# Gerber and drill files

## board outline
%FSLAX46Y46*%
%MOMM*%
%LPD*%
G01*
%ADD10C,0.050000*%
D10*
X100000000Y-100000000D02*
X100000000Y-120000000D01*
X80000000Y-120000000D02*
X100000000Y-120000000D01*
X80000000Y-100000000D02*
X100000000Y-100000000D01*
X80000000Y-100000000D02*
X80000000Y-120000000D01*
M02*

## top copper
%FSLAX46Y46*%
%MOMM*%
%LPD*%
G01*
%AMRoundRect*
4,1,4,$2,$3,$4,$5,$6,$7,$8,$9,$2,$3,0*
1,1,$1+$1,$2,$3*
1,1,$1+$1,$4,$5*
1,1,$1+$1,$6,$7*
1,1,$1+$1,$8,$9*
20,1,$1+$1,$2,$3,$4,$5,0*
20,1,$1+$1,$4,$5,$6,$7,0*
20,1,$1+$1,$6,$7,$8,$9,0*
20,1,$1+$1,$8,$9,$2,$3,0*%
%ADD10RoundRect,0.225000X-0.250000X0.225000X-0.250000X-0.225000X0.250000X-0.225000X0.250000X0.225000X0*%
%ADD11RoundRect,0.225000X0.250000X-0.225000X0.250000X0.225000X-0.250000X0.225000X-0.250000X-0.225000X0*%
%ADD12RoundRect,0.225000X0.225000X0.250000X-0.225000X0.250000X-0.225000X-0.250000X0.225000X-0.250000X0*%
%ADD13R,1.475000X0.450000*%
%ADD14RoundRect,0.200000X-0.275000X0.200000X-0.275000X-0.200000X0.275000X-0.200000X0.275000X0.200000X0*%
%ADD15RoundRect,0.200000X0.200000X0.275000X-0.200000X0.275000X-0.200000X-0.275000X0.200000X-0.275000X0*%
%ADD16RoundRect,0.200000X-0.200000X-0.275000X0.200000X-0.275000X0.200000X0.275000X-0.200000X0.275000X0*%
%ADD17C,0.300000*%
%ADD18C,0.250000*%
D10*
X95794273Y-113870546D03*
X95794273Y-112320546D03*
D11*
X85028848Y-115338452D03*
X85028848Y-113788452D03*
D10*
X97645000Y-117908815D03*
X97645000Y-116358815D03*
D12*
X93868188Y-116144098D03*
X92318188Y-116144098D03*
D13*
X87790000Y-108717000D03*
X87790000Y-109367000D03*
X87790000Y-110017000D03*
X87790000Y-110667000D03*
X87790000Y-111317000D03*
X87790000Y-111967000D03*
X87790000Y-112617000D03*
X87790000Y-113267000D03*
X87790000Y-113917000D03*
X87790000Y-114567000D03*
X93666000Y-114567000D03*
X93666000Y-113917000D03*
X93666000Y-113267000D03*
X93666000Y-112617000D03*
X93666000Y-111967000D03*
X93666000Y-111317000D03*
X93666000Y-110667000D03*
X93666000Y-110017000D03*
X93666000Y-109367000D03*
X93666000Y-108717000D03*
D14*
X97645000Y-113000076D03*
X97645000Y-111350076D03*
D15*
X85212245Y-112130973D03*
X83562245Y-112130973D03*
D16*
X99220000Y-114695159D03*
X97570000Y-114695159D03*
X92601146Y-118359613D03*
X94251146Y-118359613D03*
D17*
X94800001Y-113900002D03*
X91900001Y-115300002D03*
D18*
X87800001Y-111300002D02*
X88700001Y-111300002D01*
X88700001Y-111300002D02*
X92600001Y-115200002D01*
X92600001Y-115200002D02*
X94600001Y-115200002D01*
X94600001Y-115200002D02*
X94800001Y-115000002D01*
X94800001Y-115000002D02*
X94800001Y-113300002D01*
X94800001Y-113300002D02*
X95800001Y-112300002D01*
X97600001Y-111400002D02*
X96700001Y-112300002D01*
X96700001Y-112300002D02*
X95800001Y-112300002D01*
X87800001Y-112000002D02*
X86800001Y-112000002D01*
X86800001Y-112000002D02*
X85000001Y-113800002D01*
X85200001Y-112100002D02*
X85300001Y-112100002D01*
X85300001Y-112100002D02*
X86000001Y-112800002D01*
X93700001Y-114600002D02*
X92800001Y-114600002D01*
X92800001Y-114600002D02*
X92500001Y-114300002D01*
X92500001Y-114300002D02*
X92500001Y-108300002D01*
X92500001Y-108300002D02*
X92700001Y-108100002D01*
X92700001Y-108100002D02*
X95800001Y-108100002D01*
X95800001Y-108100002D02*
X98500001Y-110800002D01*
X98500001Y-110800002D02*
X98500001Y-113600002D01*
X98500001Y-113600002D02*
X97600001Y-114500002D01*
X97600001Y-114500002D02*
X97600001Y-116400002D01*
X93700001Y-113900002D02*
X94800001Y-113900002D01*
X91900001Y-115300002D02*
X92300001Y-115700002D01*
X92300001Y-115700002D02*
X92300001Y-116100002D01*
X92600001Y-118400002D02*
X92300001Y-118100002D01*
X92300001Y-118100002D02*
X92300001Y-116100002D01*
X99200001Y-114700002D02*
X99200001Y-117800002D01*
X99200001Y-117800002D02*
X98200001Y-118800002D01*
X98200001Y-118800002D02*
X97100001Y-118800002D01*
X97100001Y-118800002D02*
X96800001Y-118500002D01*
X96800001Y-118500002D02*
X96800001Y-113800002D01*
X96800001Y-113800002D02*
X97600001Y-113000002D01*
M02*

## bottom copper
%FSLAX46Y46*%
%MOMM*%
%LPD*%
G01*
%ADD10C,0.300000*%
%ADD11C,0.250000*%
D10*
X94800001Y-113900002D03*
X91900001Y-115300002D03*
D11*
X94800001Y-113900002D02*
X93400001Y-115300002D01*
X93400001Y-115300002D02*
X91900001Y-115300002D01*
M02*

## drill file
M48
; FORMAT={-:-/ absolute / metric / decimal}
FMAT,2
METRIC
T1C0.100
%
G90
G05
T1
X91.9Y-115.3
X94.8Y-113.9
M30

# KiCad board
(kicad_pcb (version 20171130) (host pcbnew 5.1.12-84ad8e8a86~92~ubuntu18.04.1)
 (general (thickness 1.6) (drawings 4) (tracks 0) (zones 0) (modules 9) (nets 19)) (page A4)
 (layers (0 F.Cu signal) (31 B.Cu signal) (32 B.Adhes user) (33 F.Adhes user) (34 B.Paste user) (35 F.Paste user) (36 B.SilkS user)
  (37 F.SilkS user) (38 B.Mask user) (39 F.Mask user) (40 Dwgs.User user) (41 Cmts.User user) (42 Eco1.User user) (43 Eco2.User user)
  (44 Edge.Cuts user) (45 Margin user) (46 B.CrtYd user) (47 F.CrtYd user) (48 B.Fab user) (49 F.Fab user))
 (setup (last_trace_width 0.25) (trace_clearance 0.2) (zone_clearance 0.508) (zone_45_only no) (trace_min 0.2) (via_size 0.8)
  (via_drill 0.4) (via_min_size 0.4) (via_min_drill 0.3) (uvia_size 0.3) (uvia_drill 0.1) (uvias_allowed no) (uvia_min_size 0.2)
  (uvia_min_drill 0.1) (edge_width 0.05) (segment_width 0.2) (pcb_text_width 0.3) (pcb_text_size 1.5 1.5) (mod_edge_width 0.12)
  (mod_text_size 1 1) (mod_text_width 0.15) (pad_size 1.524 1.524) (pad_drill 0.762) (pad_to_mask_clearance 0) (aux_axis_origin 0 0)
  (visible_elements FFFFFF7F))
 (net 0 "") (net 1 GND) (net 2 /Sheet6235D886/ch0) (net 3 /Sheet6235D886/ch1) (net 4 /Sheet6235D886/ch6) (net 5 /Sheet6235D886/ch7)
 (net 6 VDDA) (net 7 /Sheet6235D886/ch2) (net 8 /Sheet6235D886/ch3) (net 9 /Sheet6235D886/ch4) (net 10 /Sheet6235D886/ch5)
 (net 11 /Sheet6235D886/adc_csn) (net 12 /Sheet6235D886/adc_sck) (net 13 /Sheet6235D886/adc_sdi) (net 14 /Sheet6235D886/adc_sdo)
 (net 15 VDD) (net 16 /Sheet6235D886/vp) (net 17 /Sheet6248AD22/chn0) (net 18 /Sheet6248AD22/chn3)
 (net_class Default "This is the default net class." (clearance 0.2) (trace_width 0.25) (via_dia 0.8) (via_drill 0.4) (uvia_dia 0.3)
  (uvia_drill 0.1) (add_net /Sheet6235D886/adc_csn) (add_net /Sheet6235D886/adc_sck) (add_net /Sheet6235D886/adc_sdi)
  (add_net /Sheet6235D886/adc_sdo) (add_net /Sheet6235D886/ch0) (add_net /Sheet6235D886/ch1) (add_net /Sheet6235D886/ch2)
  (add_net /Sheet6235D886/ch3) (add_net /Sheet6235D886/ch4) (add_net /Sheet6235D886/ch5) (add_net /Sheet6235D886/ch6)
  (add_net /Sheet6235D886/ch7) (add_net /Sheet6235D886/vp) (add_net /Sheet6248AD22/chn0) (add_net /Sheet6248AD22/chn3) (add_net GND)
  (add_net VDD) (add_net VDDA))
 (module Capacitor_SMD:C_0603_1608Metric (layer F.Cu) (at 95.794273 113.095546 270.000000)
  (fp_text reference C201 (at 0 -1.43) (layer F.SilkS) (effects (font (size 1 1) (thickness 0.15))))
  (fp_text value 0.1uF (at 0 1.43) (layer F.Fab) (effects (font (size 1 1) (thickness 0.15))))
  (pad 2 smd roundrect (at 0.775 0 270.000000) (size 0.9 0.95) (layers F.Cu F.Mask F.Paste) (roundrect_rratio 0.25) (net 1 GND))
  (pad 1 smd roundrect (at -0.775 0 270.000000) (size 0.9 0.95) (layers F.Cu F.Mask F.Paste) (roundrect_rratio 0.25)
   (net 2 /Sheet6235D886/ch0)))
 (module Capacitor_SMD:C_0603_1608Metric (layer F.Cu) (at 85.028848 114.563452 90.000000)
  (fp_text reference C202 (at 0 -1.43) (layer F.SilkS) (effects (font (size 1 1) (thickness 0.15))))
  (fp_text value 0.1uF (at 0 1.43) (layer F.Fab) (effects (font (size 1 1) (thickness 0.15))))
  (pad 1 smd roundrect (at -0.775 0 90.000000) (size 0.9 0.95) (layers F.Cu F.Mask F.Paste) (roundrect_rratio 0.25) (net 1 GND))
  (pad 2 smd roundrect (at 0.775 0 90.000000) (size 0.9 0.95) (layers F.Cu F.Mask F.Paste) (roundrect_rratio 0.25)
   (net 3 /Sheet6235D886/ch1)))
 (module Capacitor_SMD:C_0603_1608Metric (layer F.Cu) (at 97.645000 117.133815 270.000000)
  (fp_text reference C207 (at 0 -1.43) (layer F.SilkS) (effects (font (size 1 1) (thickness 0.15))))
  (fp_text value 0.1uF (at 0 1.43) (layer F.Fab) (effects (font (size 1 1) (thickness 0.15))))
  (pad 2 smd roundrect (at 0.775 0 270.000000) (size 0.9 0.95) (layers F.Cu F.Mask F.Paste) (roundrect_rratio 0.25) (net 1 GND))
  (pad 1 smd roundrect (at -0.775 0 270.000000) (size 0.9 0.95) (layers F.Cu F.Mask F.Paste) (roundrect_rratio 0.25)
   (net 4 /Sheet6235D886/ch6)))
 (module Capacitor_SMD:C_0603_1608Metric (layer F.Cu) (at 93.093188 116.144098 180.000000)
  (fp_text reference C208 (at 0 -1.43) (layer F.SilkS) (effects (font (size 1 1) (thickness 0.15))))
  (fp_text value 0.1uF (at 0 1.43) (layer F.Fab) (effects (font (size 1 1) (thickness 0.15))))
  (pad 1 smd roundrect (at -0.775 0 180.000000) (size 0.9 0.95) (layers F.Cu F.Mask F.Paste) (roundrect_rratio 0.25) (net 1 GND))
  (pad 2 smd roundrect (at 0.775 0 180.000000) (size 0.9 0.95) (layers F.Cu F.Mask F.Paste) (roundrect_rratio 0.25)
   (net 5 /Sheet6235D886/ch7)))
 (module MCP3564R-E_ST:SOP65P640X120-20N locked (layer F.Cu) (at 90.728000 111.642000)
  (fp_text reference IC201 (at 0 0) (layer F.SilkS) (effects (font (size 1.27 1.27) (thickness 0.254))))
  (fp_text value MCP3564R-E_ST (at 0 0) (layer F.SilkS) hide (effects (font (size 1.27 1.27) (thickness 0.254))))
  (pad 1 smd rect (at -2.938 -2.925 90.000000) (size 0.45 1.475) (layers F.Cu F.Mask F.Paste) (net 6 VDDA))
  (pad 2 smd rect (at -2.938 -2.275 90.000000) (size 0.45 1.475) (layers F.Cu F.Mask F.Paste) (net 1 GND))
  (pad 3 smd rect (at -2.938 -1.625 90.000000) (size 0.45 1.475) (layers F.Cu F.Mask F.Paste) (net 1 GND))
  (pad 4 smd rect (at -2.938 -0.975 90.000000) (size 0.45 1.475) (layers F.Cu F.Mask F.Paste))
  (pad 5 smd rect (at -2.938 -0.325 90.000000) (size 0.45 1.475) (layers F.Cu F.Mask F.Paste) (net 2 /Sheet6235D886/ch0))
  (pad 6 smd rect (at -2.938 0.325 90.000000) (size 0.45 1.475) (layers F.Cu F.Mask F.Paste) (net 3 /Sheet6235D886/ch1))
  (pad 7 smd rect (at -2.938 0.975 90.000000) (size 0.45 1.475) (layers F.Cu F.Mask F.Paste) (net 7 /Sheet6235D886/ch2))
  (pad 8 smd rect (at -2.938 1.625 90.000000) (size 0.45 1.475) (layers F.Cu F.Mask F.Paste) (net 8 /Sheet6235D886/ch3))
  (pad 9 smd rect (at -2.938 2.275 90.000000) (size 0.45 1.475) (layers F.Cu F.Mask F.Paste) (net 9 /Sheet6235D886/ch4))
  (pad 10 smd rect (at -2.938 2.925 90.000000) (size 0.45 1.475) (layers F.Cu F.Mask F.Paste) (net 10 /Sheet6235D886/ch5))
  (pad 11 smd rect (at 2.938 2.925 90.000000) (size 0.45 1.475) (layers F.Cu F.Mask F.Paste) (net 4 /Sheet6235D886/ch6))
  (pad 12 smd rect (at 2.938 2.275 90.000000) (size 0.45 1.475) (layers F.Cu F.Mask F.Paste) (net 5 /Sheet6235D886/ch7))
  (pad 13 smd rect (at 2.938 1.625 90.000000) (size 0.45 1.475) (layers F.Cu F.Mask F.Paste) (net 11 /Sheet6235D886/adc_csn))
  (pad 14 smd rect (at 2.938 0.975 90.000000) (size 0.45 1.475) (layers F.Cu F.Mask F.Paste) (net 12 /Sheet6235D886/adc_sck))
  (pad 15 smd rect (at 2.938 0.325 90.000000) (size 0.45 1.475) (layers F.Cu F.Mask F.Paste) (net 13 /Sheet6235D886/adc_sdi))
  (pad 16 smd rect (at 2.938 -0.325 90.000000) (size 0.45 1.475) (layers F.Cu F.Mask F.Paste) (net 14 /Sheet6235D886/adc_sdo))
  (pad 17 smd rect (at 2.938 -0.975 90.000000) (size 0.45 1.475) (layers F.Cu F.Mask F.Paste))
  (pad 18 smd rect (at 2.938 -1.625 90.000000) (size 0.45 1.475) (layers F.Cu F.Mask F.Paste))
  (pad 19 smd rect (at 2.938 -2.275 90.000000) (size 0.45 1.475) (layers F.Cu F.Mask F.Paste) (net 1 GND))
  (pad 20 smd rect (at 2.938 -2.925 90.000000) (size 0.45 1.475) (layers F.Cu F.Mask F.Paste) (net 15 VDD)))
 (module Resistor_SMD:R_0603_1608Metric (layer F.Cu) (at 97.645000 112.175076 270.000000)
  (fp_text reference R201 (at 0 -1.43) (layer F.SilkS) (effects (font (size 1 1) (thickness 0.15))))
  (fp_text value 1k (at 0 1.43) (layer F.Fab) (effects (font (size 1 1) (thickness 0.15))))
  (pad 2 smd roundrect (at 0.825 0 270.000000) (size 0.8 0.95) (layers F.Cu F.Mask F.Paste) (roundrect_rratio 0.25)
   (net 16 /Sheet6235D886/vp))
  (pad 1 smd roundrect (at -0.825 0 270.000000) (size 0.8 0.95) (layers F.Cu F.Mask F.Paste) (roundrect_rratio 0.25)
   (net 2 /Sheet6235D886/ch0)))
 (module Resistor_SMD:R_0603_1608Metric (layer F.Cu) (at 84.387245 112.130973 180.000000)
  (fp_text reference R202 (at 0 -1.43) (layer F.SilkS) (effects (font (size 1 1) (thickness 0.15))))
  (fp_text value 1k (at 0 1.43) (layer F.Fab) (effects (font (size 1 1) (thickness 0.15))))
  (pad 1 smd roundrect (at -0.825 0 180.000000) (size 0.8 0.95) (layers F.Cu F.Mask F.Paste) (roundrect_rratio 0.25)
   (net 3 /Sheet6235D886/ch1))
  (pad 2 smd roundrect (at 0.825 0 180.000000) (size 0.8 0.95) (layers F.Cu F.Mask F.Paste) (roundrect_rratio 0.25)
   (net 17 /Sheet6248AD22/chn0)))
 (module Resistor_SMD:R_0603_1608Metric (layer F.Cu) (at 98.395000 114.695159)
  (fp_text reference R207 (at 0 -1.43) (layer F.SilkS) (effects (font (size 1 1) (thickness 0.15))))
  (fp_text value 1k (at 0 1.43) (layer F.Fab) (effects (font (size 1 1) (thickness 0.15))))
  (pad 2 smd roundrect (at 0.825 0) (size 0.8 0.95) (layers F.Cu F.Mask F.Paste) (roundrect_rratio 0.25) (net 16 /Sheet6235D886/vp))
  (pad 1 smd roundrect (at -0.825 0) (size 0.8 0.95) (layers F.Cu F.Mask F.Paste) (roundrect_rratio 0.25) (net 4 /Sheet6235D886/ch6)))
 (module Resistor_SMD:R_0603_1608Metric (layer F.Cu) (at 93.426146 118.359613)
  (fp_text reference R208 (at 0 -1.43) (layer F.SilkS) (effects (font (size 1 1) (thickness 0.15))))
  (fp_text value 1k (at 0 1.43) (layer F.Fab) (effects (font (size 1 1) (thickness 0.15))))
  (pad 1 smd roundrect (at -0.825 0) (size 0.8 0.95) (layers F.Cu F.Mask F.Paste) (roundrect_rratio 0.25) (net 5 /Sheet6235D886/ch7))
  (pad 2 smd roundrect (at 0.825 0) (size 0.8 0.95) (layers F.Cu F.Mask F.Paste) (roundrect_rratio 0.25) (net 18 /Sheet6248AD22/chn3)))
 (gr_line (start 100 100) (end 100 120) (layer Edge.Cuts) (width 0.05))
 (gr_line (start 80 120) (end 100 120) (layer Edge.Cuts) (width 0.05))
 (gr_line (start 80 100) (end 100 100) (layer Edge.Cuts) (width 0.05))
 (gr_line (start 80 100) (end 80 120) (layer Edge.Cuts) (width 0.05))
 (segment (start 87.800001 111.300002) (end 88.700001 111.300002) (width 0.250000) (layer F.Cu) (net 2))
 (segment (start 88.700001 111.300002) (end 92.600001 115.200002) (width 0.250000) (layer F.Cu) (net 2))
 (segment (start 92.600001 115.200002) (end 94.600001 115.200002) (width 0.250000) (layer F.Cu) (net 2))
 (segment (start 94.600001 115.200002) (end 94.800001 115.000002) (width 0.250000) (layer F.Cu) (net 2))
 (segment (start 94.800001 115.000002) (end 94.800001 113.300002) (width 0.250000) (layer F.Cu) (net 2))
 (segment (start 94.800001 113.300002) (end 95.800001 112.300002) (width 0.250000) (layer F.Cu) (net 2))
 (segment (start 97.600001 111.400002) (end 96.700001 112.300002) (width 0.250000) (layer F.Cu) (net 2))
 (segment (start 96.700001 112.300002) (end 95.800001 112.300002) (width 0.250000) (layer F.Cu) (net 2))
 (segment (start 87.800001 112.000002) (end 86.800001 112.000002) (width 0.250000) (layer F.Cu) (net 3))
 (segment (start 86.800001 112.000002) (end 85.000001 113.800002) (width 0.250000) (layer F.Cu) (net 3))
 (segment (start 85.200001 112.100002) (end 85.300001 112.100002) (width 0.250000) (layer F.Cu) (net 3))
 (segment (start 85.300001 112.100002) (end 86.000001 112.800002) (width 0.250000) (layer F.Cu) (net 3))
 (segment (start 93.700001 114.600002) (end 92.800001 114.600002) (width 0.250000) (layer F.Cu) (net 4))
 (segment (start 92.800001 114.600002) (end 92.500001 114.300002) (width 0.250000) (layer F.Cu) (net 4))
 (segment (start 92.500001 114.300002) (end 92.500001 108.300002) (width 0.250000) (layer F.Cu) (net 4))
 (segment (start 92.500001 108.300002) (end 92.700001 108.100002) (width 0.250000) (layer F.Cu) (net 4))
 (segment (start 92.700001 108.100002) (end 95.800001 108.100002) (width 0.250000) (layer F.Cu) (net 4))
 (segment (start 95.800001 108.100002) (end 98.500001 110.800002) (width 0.250000) (layer F.Cu) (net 4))
 (segment (start 98.500001 110.800002) (end 98.500001 113.600002) (width 0.250000) (layer F.Cu) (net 4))
 (segment (start 98.500001 113.600002) (end 97.600001 114.500002) (width 0.250000) (layer F.Cu) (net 4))
 (segment (start 97.600001 114.500002) (end 97.600001 116.400002) (width 0.250000) (layer F.Cu) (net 4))
 (segment (start 93.700001 113.900002) (end 94.800001 113.900002) (width 0.250000) (layer F.Cu) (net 5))
 (segment (start 94.800001 113.900002) (end 93.400001 115.300002) (width 0.250000) (layer B.Cu) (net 5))
 (segment (start 93.400001 115.300002) (end 91.900001 115.300002) (width 0.250000) (layer B.Cu) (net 5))
 (segment (start 91.900001 115.300002) (end 92.300001 115.700002) (width 0.250000) (layer F.Cu) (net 5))
 (segment (start 92.300001 115.700002) (end 92.300001 116.100002) (width 0.250000) (layer F.Cu) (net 5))
 (segment (start 92.600001 118.400002) (end 92.300001 118.100002) (width 0.250000) (layer F.Cu) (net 5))
 (segment (start 92.300001 118.100002) (end 92.300001 116.100002) (width 0.250000) (layer F.Cu) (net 5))
 (via micro (at 94.800001 113.900002) (size 0.300000) (drill 0.100000) (layers F.Cu B.Cu) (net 5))
 (via micro (at 91.900001 115.300002) (size 0.300000) (drill 0.100000) (layers F.Cu B.Cu) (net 5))
 (segment (start 99.200001 114.700002) (end 99.200001 117.800002) (width 0.250000) (layer F.Cu) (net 16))
 (segment (start 99.200001 117.800002) (end 98.200001 118.800002) (width 0.250000) (layer F.Cu) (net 16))
 (segment (start 98.200001 118.800002) (end 97.100001 118.800002) (width 0.250000) (layer F.Cu) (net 16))
 (segment (start 97.100001 118.800002) (end 96.800001 118.500002) (width 0.250000) (layer F.Cu) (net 16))
 (segment (start 96.800001 118.500002) (end 96.800001 113.800002) (width 0.250000) (layer F.Cu) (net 16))
 (segment (start 96.800001 113.800002) (end 97.600001 113.000002) (width 0.250000) (layer F.Cu) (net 16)))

